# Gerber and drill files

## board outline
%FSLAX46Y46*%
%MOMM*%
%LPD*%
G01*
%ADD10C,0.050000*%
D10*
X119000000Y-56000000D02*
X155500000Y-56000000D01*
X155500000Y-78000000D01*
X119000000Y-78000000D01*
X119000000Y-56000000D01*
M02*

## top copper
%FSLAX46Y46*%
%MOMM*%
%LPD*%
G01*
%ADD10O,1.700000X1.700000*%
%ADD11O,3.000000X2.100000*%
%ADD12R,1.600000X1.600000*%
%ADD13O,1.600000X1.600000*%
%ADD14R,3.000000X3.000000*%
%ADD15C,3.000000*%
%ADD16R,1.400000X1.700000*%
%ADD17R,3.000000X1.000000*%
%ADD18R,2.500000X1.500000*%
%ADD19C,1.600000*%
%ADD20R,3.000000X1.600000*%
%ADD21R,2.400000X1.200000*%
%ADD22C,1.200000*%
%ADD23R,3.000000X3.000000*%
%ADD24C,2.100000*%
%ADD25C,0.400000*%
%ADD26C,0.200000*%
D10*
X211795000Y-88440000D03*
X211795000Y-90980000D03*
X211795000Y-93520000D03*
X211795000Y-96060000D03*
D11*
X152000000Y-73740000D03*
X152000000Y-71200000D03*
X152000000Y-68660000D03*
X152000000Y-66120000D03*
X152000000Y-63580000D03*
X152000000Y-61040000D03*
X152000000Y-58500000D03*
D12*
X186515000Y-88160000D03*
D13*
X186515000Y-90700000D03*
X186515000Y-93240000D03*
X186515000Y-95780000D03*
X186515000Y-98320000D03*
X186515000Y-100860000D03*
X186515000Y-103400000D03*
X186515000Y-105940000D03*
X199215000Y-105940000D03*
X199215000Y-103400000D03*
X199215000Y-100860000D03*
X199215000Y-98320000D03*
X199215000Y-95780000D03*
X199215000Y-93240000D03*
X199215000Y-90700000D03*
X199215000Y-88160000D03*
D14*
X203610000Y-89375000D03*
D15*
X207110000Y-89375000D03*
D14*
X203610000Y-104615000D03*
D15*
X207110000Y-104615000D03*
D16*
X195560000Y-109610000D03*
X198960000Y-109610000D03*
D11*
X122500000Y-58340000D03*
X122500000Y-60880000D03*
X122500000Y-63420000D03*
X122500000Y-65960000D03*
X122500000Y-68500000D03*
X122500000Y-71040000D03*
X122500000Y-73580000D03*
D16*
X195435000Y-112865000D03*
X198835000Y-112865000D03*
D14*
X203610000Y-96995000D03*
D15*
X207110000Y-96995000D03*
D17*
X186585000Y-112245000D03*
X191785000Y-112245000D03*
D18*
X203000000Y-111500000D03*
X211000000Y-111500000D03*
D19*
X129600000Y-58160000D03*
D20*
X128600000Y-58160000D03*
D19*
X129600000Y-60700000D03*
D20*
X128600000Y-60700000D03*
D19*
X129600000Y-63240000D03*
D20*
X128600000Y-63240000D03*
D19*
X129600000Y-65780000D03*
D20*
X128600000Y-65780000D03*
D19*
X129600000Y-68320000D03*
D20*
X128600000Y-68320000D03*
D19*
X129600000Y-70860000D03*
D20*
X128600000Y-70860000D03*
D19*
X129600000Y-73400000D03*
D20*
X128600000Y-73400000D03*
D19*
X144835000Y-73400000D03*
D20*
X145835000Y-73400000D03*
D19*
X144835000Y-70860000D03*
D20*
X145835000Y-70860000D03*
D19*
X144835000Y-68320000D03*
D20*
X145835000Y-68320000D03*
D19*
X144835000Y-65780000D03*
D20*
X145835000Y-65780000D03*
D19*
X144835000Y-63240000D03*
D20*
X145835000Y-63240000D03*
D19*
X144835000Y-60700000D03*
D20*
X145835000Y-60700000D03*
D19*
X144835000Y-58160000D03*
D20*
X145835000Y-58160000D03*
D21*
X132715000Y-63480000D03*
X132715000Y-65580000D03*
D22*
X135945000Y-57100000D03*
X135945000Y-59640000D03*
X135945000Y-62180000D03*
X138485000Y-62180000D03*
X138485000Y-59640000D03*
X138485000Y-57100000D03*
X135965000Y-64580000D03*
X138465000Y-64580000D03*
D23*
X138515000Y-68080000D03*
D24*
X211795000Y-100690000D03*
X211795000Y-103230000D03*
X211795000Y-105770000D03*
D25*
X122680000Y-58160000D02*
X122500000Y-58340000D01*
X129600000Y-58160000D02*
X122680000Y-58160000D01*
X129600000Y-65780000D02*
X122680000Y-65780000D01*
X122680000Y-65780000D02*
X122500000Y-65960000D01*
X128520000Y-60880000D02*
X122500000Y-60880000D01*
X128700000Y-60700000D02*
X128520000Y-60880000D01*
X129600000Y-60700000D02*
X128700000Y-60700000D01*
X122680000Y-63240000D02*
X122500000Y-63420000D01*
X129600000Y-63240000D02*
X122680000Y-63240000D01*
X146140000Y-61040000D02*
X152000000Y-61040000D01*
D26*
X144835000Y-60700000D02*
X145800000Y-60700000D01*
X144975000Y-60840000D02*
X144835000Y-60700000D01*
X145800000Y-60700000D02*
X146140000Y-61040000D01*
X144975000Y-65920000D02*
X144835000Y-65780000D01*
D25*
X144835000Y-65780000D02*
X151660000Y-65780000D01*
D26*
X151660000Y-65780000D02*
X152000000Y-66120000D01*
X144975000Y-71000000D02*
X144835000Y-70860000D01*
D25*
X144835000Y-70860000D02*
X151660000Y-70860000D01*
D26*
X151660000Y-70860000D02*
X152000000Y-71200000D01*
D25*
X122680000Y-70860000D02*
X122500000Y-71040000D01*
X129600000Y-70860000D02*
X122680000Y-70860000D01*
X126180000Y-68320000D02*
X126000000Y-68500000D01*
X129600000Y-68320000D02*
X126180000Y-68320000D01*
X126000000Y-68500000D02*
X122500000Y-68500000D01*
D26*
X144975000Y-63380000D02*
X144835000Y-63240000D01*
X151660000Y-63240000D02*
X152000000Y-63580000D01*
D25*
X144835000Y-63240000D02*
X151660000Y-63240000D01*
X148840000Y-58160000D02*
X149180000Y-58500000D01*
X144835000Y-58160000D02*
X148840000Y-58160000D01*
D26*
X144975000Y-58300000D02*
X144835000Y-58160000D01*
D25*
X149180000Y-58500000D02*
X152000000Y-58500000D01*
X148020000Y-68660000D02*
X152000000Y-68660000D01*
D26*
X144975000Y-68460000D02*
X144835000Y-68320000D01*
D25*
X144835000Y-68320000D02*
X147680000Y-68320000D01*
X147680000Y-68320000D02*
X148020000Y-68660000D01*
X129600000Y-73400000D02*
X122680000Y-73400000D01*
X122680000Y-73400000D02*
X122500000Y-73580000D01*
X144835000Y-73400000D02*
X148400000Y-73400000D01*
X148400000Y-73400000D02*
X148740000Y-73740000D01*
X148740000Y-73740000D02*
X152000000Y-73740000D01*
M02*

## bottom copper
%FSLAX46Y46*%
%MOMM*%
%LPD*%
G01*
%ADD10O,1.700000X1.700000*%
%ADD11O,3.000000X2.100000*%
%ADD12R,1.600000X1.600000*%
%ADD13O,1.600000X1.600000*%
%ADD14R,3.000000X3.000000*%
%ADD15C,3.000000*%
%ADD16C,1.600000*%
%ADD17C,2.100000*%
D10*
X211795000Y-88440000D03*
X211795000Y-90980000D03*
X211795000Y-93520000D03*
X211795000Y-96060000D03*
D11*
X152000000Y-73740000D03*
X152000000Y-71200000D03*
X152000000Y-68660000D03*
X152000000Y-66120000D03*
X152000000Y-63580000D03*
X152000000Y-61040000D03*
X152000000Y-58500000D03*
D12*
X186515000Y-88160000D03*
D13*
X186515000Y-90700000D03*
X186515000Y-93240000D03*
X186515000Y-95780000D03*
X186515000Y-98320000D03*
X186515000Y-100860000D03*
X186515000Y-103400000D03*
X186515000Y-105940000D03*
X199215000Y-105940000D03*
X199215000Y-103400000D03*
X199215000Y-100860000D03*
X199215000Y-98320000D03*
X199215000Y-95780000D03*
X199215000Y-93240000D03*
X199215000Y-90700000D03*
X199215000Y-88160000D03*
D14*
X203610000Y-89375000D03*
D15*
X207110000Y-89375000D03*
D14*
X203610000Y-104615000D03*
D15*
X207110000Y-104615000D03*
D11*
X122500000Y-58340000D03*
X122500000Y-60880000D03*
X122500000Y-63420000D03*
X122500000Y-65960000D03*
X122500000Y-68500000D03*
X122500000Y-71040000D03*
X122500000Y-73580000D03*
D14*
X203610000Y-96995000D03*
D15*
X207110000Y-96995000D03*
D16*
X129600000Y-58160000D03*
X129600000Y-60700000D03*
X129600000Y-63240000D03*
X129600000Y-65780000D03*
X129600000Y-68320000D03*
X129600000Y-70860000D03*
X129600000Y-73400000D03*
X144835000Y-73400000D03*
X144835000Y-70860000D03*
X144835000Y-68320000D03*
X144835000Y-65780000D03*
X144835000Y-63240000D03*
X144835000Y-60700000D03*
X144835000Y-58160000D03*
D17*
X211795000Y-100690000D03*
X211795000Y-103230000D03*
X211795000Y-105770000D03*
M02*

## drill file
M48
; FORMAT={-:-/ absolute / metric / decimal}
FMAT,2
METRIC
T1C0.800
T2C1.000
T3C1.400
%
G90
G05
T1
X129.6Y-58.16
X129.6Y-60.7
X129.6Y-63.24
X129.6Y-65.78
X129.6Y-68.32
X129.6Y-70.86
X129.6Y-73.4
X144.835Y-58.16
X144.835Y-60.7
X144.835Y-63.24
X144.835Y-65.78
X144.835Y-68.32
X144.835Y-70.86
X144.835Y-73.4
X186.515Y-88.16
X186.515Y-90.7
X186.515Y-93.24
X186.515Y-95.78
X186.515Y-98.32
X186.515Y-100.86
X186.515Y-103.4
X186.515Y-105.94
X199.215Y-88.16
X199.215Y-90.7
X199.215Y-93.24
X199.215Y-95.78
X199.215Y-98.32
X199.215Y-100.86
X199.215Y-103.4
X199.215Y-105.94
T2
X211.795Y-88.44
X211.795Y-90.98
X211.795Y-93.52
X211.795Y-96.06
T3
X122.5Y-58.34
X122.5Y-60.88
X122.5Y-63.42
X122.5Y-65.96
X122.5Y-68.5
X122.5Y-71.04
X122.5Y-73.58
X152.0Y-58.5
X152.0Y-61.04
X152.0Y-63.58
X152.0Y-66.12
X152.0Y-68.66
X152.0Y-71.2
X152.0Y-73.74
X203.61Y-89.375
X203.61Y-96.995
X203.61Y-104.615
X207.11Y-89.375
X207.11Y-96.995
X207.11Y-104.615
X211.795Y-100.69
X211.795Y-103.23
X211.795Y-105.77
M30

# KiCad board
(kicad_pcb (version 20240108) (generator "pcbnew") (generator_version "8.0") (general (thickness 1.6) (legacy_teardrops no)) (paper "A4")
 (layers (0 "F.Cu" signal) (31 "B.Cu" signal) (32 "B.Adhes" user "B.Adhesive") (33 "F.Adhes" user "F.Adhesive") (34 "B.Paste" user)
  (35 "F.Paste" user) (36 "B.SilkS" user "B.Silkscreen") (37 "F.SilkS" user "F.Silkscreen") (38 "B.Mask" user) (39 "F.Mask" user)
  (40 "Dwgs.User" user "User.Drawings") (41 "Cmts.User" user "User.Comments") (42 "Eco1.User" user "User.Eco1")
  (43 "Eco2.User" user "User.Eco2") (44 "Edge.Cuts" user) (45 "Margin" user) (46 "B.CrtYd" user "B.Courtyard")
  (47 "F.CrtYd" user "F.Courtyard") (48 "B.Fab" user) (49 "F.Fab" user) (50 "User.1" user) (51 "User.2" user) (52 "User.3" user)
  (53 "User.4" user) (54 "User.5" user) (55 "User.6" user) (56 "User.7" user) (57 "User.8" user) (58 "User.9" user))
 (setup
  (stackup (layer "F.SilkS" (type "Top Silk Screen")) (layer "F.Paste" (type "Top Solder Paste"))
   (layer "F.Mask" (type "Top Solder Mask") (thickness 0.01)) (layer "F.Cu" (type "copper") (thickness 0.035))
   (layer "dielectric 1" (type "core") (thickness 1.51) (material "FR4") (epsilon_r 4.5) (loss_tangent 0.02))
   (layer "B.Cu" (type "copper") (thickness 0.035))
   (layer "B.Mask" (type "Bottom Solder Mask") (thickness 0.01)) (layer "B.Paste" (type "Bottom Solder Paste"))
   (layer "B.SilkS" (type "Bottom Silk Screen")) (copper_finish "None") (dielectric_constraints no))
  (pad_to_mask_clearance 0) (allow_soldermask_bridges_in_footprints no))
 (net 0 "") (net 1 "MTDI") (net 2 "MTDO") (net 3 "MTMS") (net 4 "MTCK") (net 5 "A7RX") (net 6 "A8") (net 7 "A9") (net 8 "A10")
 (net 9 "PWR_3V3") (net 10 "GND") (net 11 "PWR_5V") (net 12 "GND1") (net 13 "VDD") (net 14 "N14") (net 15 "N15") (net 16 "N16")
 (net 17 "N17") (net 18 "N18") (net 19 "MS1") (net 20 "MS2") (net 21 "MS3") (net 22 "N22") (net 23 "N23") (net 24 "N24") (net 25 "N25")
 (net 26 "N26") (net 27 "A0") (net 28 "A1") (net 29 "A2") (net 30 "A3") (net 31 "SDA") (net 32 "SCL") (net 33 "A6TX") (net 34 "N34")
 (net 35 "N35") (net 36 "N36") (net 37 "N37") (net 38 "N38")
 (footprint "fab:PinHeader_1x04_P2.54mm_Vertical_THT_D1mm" (layer "F.Cu") (at 211.795 88.44)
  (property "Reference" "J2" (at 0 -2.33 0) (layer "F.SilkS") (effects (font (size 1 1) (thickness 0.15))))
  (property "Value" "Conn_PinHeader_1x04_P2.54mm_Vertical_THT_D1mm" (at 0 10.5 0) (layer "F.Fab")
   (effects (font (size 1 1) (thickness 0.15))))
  (pad "1" thru_hole oval (at 0 0) (size 1.7 1.7) (drill 1) (layers "*.Cu" "*.Mask") (remove_unused_layers no) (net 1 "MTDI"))
  (pad "2" thru_hole oval (at 0 2.54) (size 1.7 1.7) (drill 1) (layers "*.Cu" "*.Mask") (remove_unused_layers no) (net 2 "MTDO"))
  (pad "3" thru_hole oval (at 0 5.08) (size 1.7 1.7) (drill 1) (layers "*.Cu" "*.Mask") (remove_unused_layers no) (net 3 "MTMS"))
  (pad "4" thru_hole oval (at 0 7.62) (size 1.7 1.7) (drill 1) (layers "*.Cu" "*.Mask") (remove_unused_layers no) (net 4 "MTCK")))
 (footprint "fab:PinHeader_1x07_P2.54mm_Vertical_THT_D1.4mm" (layer "F.Cu") (at 152 73.74 180)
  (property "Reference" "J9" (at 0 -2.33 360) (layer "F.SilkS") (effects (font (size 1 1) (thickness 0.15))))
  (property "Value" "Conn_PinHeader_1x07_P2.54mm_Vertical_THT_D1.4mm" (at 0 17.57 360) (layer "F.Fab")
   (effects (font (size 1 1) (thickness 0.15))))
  (pad "1" thru_hole oval (at 0 0 180) (size 3 2.1) (drill 1.4) (layers "*.Cu" "*.Mask") (remove_unused_layers no) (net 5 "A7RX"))
  (pad "2" thru_hole oval (at 0 2.54 180) (size 3 2.1) (drill 1.4) (layers "*.Cu" "*.Mask") (remove_unused_layers no) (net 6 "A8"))
  (pad "3" thru_hole oval (at 0 5.08 180) (size 3 2.1) (drill 1.4) (layers "*.Cu" "*.Mask") (remove_unused_layers no) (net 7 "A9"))
  (pad "4" thru_hole oval (at 0 7.62 180) (size 3 2.1) (drill 1.4) (layers "*.Cu" "*.Mask") (remove_unused_layers no) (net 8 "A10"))
  (pad "5" thru_hole oval (at 0 10.16 180) (size 3 2.1) (drill 1.4) (layers "*.Cu" "*.Mask") (remove_unused_layers no) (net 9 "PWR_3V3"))
  (pad "6" thru_hole oval (at 0 12.7 180) (size 3 2.1) (drill 1.4) (layers "*.Cu" "*.Mask") (remove_unused_layers no) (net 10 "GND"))
  (pad "7" thru_hole oval (at 0 15.24 180) (size 3 2.1) (drill 1.4) (layers "*.Cu" "*.Mask") (remove_unused_layers no) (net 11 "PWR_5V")))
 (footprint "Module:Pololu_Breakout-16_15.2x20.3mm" (layer "F.Cu") (at 186.515 88.16)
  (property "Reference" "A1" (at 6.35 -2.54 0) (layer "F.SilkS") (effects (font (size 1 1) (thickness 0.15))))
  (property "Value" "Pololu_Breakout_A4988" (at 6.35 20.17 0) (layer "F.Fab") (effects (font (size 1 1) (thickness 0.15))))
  (pad "1" thru_hole rect (at 0 0) (size 1.6 1.6) (drill 0.8) (layers "*.Cu" "*.Mask") (remove_unused_layers no) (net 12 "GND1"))
  (pad "2" thru_hole oval (at 0 2.54) (size 1.6 1.6) (drill 0.8) (layers "*.Cu" "*.Mask") (remove_unused_layers no) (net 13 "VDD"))
  (pad "3" thru_hole oval (at 0 5.08) (size 1.6 1.6) (drill 0.8) (layers "*.Cu" "*.Mask") (remove_unused_layers no) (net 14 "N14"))
  (pad "4" thru_hole oval (at 0 7.62) (size 1.6 1.6) (drill 0.8) (layers "*.Cu" "*.Mask") (remove_unused_layers no) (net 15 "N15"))
  (pad "5" thru_hole oval (at 0 10.16) (size 1.6 1.6) (drill 0.8) (layers "*.Cu" "*.Mask") (remove_unused_layers no) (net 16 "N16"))
  (pad "6" thru_hole oval (at 0 12.7) (size 1.6 1.6) (drill 0.8) (layers "*.Cu" "*.Mask") (remove_unused_layers no) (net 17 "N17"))
  (pad "7" thru_hole oval (at 0 15.24) (size 1.6 1.6) (drill 0.8) (layers "*.Cu" "*.Mask") (remove_unused_layers no) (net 12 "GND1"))
  (pad "8" thru_hole oval (at 0 17.78) (size 1.6 1.6) (drill 0.8) (layers "*.Cu" "*.Mask") (remove_unused_layers no) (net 13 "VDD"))
  (pad "9" thru_hole oval (at 12.7 17.78) (size 1.6 1.6) (drill 0.8) (layers "*.Cu" "*.Mask") (remove_unused_layers no) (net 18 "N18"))
  (pad "10" thru_hole oval (at 12.7 15.24) (size 1.6 1.6) (drill 0.8) (layers "*.Cu" "*.Mask") (remove_unused_layers no) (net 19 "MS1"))
  (pad "11" thru_hole oval (at 12.7 12.7) (size 1.6 1.6) (drill 0.8) (layers "*.Cu" "*.Mask") (remove_unused_layers no) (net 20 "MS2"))
  (pad "12" thru_hole oval (at 12.7 10.16) (size 1.6 1.6) (drill 0.8) (layers "*.Cu" "*.Mask") (remove_unused_layers no) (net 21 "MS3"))
  (pad "13" thru_hole oval (at 12.7 7.62) (size 1.6 1.6) (drill 0.8) (layers "*.Cu" "*.Mask") (remove_unused_layers no) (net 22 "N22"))
  (pad "14" thru_hole oval (at 12.7 5.08) (size 1.6 1.6) (drill 0.8) (layers "*.Cu" "*.Mask") (remove_unused_layers no) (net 22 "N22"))
  (pad "15" thru_hole oval (at 12.7 2.54) (size 1.6 1.6) (drill 0.8) (layers "*.Cu" "*.Mask") (remove_unused_layers no) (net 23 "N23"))
  (pad "16" thru_hole oval (at 12.7 0) (size 1.6 1.6) (drill 0.8) (layers "*.Cu" "*.Mask") (remove_unused_layers no) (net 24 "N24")))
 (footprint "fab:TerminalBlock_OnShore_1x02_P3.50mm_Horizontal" (layer "F.Cu") (at 203.61 89.375)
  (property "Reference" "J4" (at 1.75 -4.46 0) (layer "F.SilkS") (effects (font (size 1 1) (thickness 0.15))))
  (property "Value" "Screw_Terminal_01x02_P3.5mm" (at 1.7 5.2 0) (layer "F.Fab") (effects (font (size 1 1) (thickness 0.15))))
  (pad "1" thru_hole rect (at 0 0) (size 3 3) (drill 1.4) (layers "*.Cu" "*.Mask") (remove_unused_layers no) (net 24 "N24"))
  (pad "2" thru_hole circle (at 3.5 0) (size 3 3) (drill 1.4) (layers "*.Cu" "*.Mask") (remove_unused_layers no) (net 23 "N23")))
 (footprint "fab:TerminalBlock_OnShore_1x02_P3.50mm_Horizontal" (layer "F.Cu") (at 203.61 104.615)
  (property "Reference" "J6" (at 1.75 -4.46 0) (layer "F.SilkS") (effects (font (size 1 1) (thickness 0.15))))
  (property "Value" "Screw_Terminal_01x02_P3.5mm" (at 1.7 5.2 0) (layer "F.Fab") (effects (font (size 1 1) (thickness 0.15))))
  (pad "1" thru_hole rect (at 0 0) (size 3 3) (drill 1.4) (layers "*.Cu" "*.Mask") (remove_unused_layers no) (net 12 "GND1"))
  (pad "2" thru_hole circle (at 3.5 0) (size 3 3) (drill 1.4) (layers "*.Cu" "*.Mask") (remove_unused_layers no) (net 13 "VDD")))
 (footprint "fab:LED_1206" (layer "F.Cu") (at 197.26 109.61)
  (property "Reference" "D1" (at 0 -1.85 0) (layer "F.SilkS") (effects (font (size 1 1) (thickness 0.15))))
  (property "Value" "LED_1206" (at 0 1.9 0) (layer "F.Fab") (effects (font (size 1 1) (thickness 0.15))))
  (pad "1" smd rect (at -1.7 0) (size 1.4 1.7) (layers "F.Cu" "F.Paste" "F.Mask") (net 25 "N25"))
  (pad "2" smd rect (at 1.7 0) (size 1.4 1.7) (layers "F.Cu" "F.Paste" "F.Mask") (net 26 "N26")))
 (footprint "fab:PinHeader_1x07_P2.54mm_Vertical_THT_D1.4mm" (layer "F.Cu") (at 122.5 58.34)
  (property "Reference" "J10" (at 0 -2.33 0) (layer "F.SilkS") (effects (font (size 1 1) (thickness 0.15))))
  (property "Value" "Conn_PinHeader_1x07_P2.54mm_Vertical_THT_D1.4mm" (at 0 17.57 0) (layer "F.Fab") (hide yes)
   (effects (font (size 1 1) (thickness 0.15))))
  (pad "1" thru_hole oval (at 0 0) (size 3 2.1) (drill 1.4) (layers "*.Cu" "*.Mask") (remove_unused_layers no) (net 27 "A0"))
  (pad "2" thru_hole oval (at 0 2.54) (size 3 2.1) (drill 1.4) (layers "*.Cu" "*.Mask") (remove_unused_layers no) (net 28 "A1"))
  (pad "3" thru_hole oval (at 0 5.08) (size 3 2.1) (drill 1.4) (layers "*.Cu" "*.Mask") (remove_unused_layers no) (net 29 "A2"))
  (pad "4" thru_hole oval (at 0 7.62) (size 3 2.1) (drill 1.4) (layers "*.Cu" "*.Mask") (remove_unused_layers no) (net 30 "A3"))
  (pad "5" thru_hole oval (at 0 10.16) (size 3 2.1) (drill 1.4) (layers "*.Cu" "*.Mask") (remove_unused_layers no) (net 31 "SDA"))
  (pad "6" thru_hole oval (at 0 12.7) (size 3 2.1) (drill 1.4) (layers "*.Cu" "*.Mask") (remove_unused_layers no) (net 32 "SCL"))
  (pad "7" thru_hole oval (at 0 15.24) (size 3 2.1) (drill 1.4) (layers "*.Cu" "*.Mask") (remove_unused_layers no) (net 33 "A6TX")))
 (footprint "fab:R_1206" (layer "F.Cu") (at 197.135 112.865)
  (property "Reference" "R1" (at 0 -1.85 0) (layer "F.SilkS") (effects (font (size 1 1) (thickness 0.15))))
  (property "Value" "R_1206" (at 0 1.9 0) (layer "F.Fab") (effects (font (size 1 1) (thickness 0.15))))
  (pad "1" smd rect (at -1.7 0) (size 1.4 1.7) (layers "F.Cu" "F.Paste" "F.Mask") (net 10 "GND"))
  (pad "2" smd rect (at 1.7 0) (size 1.4 1.7) (layers "F.Cu" "F.Paste" "F.Mask") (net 26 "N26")))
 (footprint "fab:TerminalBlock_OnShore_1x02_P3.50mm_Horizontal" (layer "F.Cu") (at 203.61 96.995)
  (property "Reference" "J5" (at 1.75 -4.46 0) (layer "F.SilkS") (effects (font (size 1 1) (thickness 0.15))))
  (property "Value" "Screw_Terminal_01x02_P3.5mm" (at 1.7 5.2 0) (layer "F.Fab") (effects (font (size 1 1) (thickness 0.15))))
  (pad "1" thru_hole rect (at 0 0) (size 3 3) (drill 1.4) (layers "*.Cu" "*.Mask") (remove_unused_layers no) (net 12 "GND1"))
  (pad "2" thru_hole circle (at 3.5 0) (size 3 3) (drill 1.4) (layers "*.Cu" "*.Mask") (remove_unused_layers no) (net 13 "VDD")))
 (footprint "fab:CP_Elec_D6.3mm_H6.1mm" (layer "F.Cu") (at 189.185 112.245)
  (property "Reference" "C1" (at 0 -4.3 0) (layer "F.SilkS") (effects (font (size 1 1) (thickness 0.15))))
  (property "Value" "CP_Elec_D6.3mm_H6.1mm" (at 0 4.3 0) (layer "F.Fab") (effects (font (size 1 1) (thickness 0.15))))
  (pad "1" smd rect (at -2.6 0) (size 3 1) (layers "F.Cu" "F.Paste" "F.Mask") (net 13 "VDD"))
  (pad "2" smd rect (at 2.6 0) (size 3 1) (layers "F.Cu" "F.Paste" "F.Mask") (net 12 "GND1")))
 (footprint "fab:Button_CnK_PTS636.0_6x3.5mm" (layer "F.Cu") (at 207 111.5)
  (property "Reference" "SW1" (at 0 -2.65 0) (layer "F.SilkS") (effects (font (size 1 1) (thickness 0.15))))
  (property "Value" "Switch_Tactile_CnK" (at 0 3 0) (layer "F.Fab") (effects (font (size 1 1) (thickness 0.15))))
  (pad "1" smd rect (at -4 0) (size 2.5 1.5) (layers "F.Cu" "F.Paste" "F.Mask") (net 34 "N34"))
  (pad "2" smd rect (at 4 0) (size 2.5 1.5) (layers "F.Cu" "F.Paste" "F.Mask") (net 25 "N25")))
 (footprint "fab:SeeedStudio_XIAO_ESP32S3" (layer "F.Cu") (at 137.215 65.78)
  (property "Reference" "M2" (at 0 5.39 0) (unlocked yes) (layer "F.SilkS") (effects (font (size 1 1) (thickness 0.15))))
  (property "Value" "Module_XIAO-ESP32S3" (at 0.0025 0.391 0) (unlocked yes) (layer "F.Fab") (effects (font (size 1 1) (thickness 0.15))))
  (pad "1" thru_hole circle (at -7.615 -7.62) (size 1.6 1.6) (drill 0.8) (layers "*.Cu" "*.Mask") (remove_unused_layers no) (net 27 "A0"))
  (pad "1" smd rect (at -7.615 -7.62) (size 3 1.6) (drill (offset -1 0)) (layers "F.Cu" "F.Paste" "F.Mask") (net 27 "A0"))
  (pad "2" thru_hole circle (at -7.615 -5.08) (size 1.6 1.6) (drill 0.8) (layers "*.Cu" "*.Mask") (remove_unused_layers no) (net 28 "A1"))
  (pad "2" smd rect (at -7.615 -5.08) (size 3 1.6) (drill (offset -1 0)) (layers "F.Cu" "F.Paste" "F.Mask") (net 28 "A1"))
  (pad "3" thru_hole circle (at -7.615 -2.54) (size 1.6 1.6) (drill 0.8) (layers "*.Cu" "*.Mask") (remove_unused_layers no) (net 29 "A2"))
  (pad "3" smd rect (at -7.615 -2.54) (size 3 1.6) (drill (offset -1 0)) (layers "F.Cu" "F.Paste" "F.Mask") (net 29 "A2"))
  (pad "4" thru_hole circle (at -7.615 0) (size 1.6 1.6) (drill 0.8) (layers "*.Cu" "*.Mask") (remove_unused_layers no) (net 30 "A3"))
  (pad "4" smd rect (at -7.615 0) (size 3 1.6) (drill (offset -1 0)) (layers "F.Cu" "F.Paste" "F.Mask") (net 30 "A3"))
  (pad "5" thru_hole circle (at -7.615 2.54) (size 1.6 1.6) (drill 0.8) (layers "*.Cu" "*.Mask") (remove_unused_layers no) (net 31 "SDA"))
  (pad "5" smd rect (at -7.615 2.54) (size 3 1.6) (drill (offset -1 0)) (layers "F.Cu" "F.Paste" "F.Mask") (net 31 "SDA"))
  (pad "6" thru_hole circle (at -7.615 5.08) (size 1.6 1.6) (drill 0.8) (layers "*.Cu" "*.Mask") (remove_unused_layers no) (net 32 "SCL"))
  (pad "6" smd rect (at -7.615 5.08) (size 3 1.6) (drill (offset -1 0)) (layers "F.Cu" "F.Paste" "F.Mask") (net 32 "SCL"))
  (pad "7" thru_hole circle (at -7.615 7.62) (size 1.6 1.6) (drill 0.8) (layers "*.Cu" "*.Mask") (remove_unused_layers no) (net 33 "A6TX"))
  (pad "7" smd rect (at -7.615 7.62) (size 3 1.6) (drill (offset -1 0)) (layers "F.Cu" "F.Paste" "F.Mask") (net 33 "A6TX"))
  (pad "8" thru_hole circle (at 7.62 7.62) (size 1.6 1.6) (drill 0.8) (layers "*.Cu" "*.Mask") (remove_unused_layers no) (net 5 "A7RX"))
  (pad "8" smd rect (at 7.62 7.62) (size 3 1.6) (drill (offset 1 0)) (layers "F.Cu" "F.Paste" "F.Mask") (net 5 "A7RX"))
  (pad "9" thru_hole circle (at 7.62 5.08) (size 1.6 1.6) (drill 0.8) (layers "*.Cu" "*.Mask") (remove_unused_layers no) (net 6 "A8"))
  (pad "9" smd rect (at 7.62 5.08) (size 3 1.6) (drill (offset 1 0)) (layers "F.Cu" "F.Paste" "F.Mask") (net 6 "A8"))
  (pad "10" thru_hole circle (at 7.62 2.54) (size 1.6 1.6) (drill 0.8) (layers "*.Cu" "*.Mask") (remove_unused_layers no) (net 7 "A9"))
  (pad "10" smd rect (at 7.62 2.54) (size 3 1.6) (drill (offset 1 0)) (layers "F.Cu" "F.Paste" "F.Mask") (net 7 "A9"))
  (pad "11" thru_hole circle (at 7.62 0) (size 1.6 1.6) (drill 0.8) (layers "*.Cu" "*.Mask") (remove_unused_layers no) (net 8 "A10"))
  (pad "11" smd rect (at 7.62 0) (size 3 1.6) (drill (offset 1 0)) (layers "F.Cu" "F.Paste" "F.Mask") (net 8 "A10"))
  (pad "12" thru_hole circle (at 7.62 -2.54) (size 1.6 1.6) (drill 0.8) (layers "*.Cu" "*.Mask") (remove_unused_layers no) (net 9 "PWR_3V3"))
  (pad "12" smd rect (at 7.62 -2.54) (size 3 1.6) (drill (offset 1 0)) (layers "F.Cu" "F.Paste" "F.Mask") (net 9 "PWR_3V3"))
  (pad "13" thru_hole circle (at 7.62 -5.08) (size 1.6 1.6) (drill 0.8) (layers "*.Cu" "*.Mask") (remove_unused_layers no) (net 10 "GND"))
  (pad "13" smd rect (at 7.62 -5.08) (size 3 1.6) (drill (offset 1 0)) (layers "F.Cu" "F.Paste" "F.Mask") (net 10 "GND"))
  (pad "14" thru_hole circle (at 7.62 -7.62) (size 1.6 1.6) (drill 0.8) (layers "*.Cu" "*.Mask") (remove_unused_layers no) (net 11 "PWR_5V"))
  (pad "14" smd rect (at 7.62 -7.62) (size 3 1.6) (drill (offset 1 0)) (layers "F.Cu" "F.Paste" "F.Mask") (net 11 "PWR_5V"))
  (pad "15" smd rect (at -4.5 -2.3) (size 2.4 1.2) (layers "F.Cu" "F.Paste" "F.Mask") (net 10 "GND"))
  (pad "16" smd rect (at -4.5 -0.2) (size 2.4 1.2) (layers "F.Cu" "F.Paste" "F.Mask") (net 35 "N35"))
  (pad "17" smd circle (at -1.27 -8.68) (size 1.2 1.2) (layers "F.Cu" "F.Paste" "F.Mask") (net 1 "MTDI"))
  (pad "18" smd circle (at -1.27 -6.14) (size 1.2 1.2) (layers "F.Cu" "F.Paste" "F.Mask") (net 34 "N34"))
  (pad "19" smd circle (at -1.27 -3.6) (size 1.2 1.2) (layers "F.Cu" "F.Paste" "F.Mask") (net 3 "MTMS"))
  (pad "20" smd circle (at 1.27 -3.6) (size 1.2 1.2) (layers "F.Cu" "F.Paste" "F.Mask") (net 4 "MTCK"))
  (pad "21" smd circle (at 1.27 -6.14) (size 1.2 1.2) (layers "F.Cu" "F.Paste" "F.Mask") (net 10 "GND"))
  (pad "22" smd circle (at 1.27 -8.68) (size 1.2 1.2) (layers "F.Cu" "F.Paste" "F.Mask") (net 2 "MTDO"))
  (pad "23" smd circle (at -1.25 -1.2) (size 1.2 1.2) (layers "F.Cu" "F.Paste" "F.Mask") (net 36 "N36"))
  (pad "24" smd circle (at 1.25 -1.2) (size 1.2 1.2) (layers "F.Cu" "F.Paste" "F.Mask") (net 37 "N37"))
  (pad "25" smd rect (at 1.3 2.3) (size 3 3) (layers "F.Cu" "F.Paste" "F.Mask") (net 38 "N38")))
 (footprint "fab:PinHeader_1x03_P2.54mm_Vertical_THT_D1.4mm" (layer "F.Cu") (at 211.795 100.69)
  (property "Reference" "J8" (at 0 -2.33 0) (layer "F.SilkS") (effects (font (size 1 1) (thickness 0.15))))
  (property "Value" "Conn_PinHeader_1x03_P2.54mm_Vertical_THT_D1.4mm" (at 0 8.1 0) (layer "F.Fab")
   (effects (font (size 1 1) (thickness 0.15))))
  (pad "1" thru_hole circle (at 0 0) (size 2.1 2.1) (drill 1.4) (layers "*.Cu" "*.Mask") (remove_unused_layers no) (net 19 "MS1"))
  (pad "2" thru_hole circle (at 0 2.54) (size 2.1 2.1) (drill 1.4) (layers "*.Cu" "*.Mask") (remove_unused_layers no) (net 20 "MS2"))
  (pad "3" thru_hole circle (at 0 5.08) (size 2.1 2.1) (drill 1.4) (layers "*.Cu" "*.Mask") (remove_unused_layers no) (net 21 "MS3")))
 (gr_rect (start 119 56) (end 155.5 78) (stroke (width 0.05) (type default)) (fill none) (layer "Edge.Cuts"))
 (segment (start 122.68 58.16) (end 122.5 58.34) (width 0.4) (layer "F.Cu") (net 27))
 (segment (start 129.6 58.16) (end 122.68 58.16) (width 0.4) (layer "F.Cu") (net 27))
 (segment (start 129.6 65.78) (end 122.68 65.78) (width 0.4) (layer "F.Cu") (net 30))
 (segment (start 122.68 65.78) (end 122.5 65.96) (width 0.4) (layer "F.Cu") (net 30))
 (segment (start 128.52 60.88) (end 122.5 60.88) (width 0.4) (layer "F.Cu") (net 28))
 (segment (start 128.7 60.7) (end 128.52 60.88) (width 0.4) (layer "F.Cu") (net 28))
 (segment (start 129.6 60.7) (end 128.7 60.7) (width 0.4) (layer "F.Cu") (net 28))
 (segment (start 122.68 63.24) (end 122.5 63.42) (width 0.4) (layer "F.Cu") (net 29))
 (segment (start 129.6 63.24) (end 122.68 63.24) (width 0.4) (layer "F.Cu") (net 29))
 (segment (start 146.14 61.04) (end 152 61.04) (width 0.4) (layer "F.Cu") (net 10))
 (segment (start 144.835 60.7) (end 145.8 60.7) (width 0.2) (layer "F.Cu") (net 10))
 (segment (start 144.975 60.84) (end 144.835 60.7) (width 0.2) (layer "F.Cu") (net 10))
 (segment (start 145.8 60.7) (end 146.14 61.04) (width 0.2) (layer "F.Cu") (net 10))
 (segment (start 144.975 65.92) (end 144.835 65.78) (width 0.2) (layer "F.Cu") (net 8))
 (segment (start 144.835 65.78) (end 151.66 65.78) (width 0.4) (layer "F.Cu") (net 8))
 (segment (start 151.66 65.78) (end 152 66.12) (width 0.2) (layer "F.Cu") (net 8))
 (segment (start 144.975 71) (end 144.835 70.86) (width 0.2) (layer "F.Cu") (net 6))
 (segment (start 144.835 70.86) (end 151.66 70.86) (width 0.4) (layer "F.Cu") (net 6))
 (segment (start 151.66 70.86) (end 152 71.2) (width 0.2) (layer "F.Cu") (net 6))
 (segment (start 122.68 70.86) (end 122.5 71.04) (width 0.4) (layer "F.Cu") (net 32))
 (segment (start 129.6 70.86) (end 122.68 70.86) (width 0.4) (layer "F.Cu") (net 32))
 (segment (start 126.18 68.32) (end 126 68.5) (width 0.4) (layer "F.Cu") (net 31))
 (segment (start 129.6 68.32) (end 126.18 68.32) (width 0.4) (layer "F.Cu") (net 31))
 (segment (start 126 68.5) (end 122.5 68.5) (width 0.4) (layer "F.Cu") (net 31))
 (segment (start 144.975 63.38) (end 144.835 63.24) (width 0.2) (layer "F.Cu") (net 9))
 (segment (start 151.66 63.24) (end 152 63.58) (width 0.2) (layer "F.Cu") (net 9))
 (segment (start 144.835 63.24) (end 151.66 63.24) (width 0.4) (layer "F.Cu") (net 9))
 (segment (start 148.84 58.16) (end 149.18 58.5) (width 0.4) (layer "F.Cu") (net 11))
 (segment (start 144.835 58.16) (end 148.84 58.16) (width 0.4) (layer "F.Cu") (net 11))
 (segment (start 144.975 58.3) (end 144.835 58.16) (width 0.2) (layer "F.Cu") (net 11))
 (segment (start 149.18 58.5) (end 152 58.5) (width 0.4) (layer "F.Cu") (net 11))
 (segment (start 148.02 68.66) (end 152 68.66) (width 0.4) (layer "F.Cu") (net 7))
 (segment (start 144.975 68.46) (end 144.835 68.32) (width 0.2) (layer "F.Cu") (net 7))
 (segment (start 144.835 68.32) (end 147.68 68.32) (width 0.4) (layer "F.Cu") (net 7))
 (segment (start 147.68 68.32) (end 148.02 68.66) (width 0.4) (layer "F.Cu") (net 7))
 (segment (start 129.6 73.4) (end 122.68 73.4) (width 0.4) (layer "F.Cu") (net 33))
 (segment (start 122.68 73.4) (end 122.5 73.58) (width 0.4) (layer "F.Cu") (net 33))
 (segment (start 144.835 73.4) (end 148.4 73.4) (width 0.4) (layer "F.Cu") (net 5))
 (segment (start 148.4 73.4) (end 148.74 73.74) (width 0.4) (layer "F.Cu") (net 5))
 (segment (start 148.74 73.74) (end 152 73.74) (width 0.4) (layer "F.Cu") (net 5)))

